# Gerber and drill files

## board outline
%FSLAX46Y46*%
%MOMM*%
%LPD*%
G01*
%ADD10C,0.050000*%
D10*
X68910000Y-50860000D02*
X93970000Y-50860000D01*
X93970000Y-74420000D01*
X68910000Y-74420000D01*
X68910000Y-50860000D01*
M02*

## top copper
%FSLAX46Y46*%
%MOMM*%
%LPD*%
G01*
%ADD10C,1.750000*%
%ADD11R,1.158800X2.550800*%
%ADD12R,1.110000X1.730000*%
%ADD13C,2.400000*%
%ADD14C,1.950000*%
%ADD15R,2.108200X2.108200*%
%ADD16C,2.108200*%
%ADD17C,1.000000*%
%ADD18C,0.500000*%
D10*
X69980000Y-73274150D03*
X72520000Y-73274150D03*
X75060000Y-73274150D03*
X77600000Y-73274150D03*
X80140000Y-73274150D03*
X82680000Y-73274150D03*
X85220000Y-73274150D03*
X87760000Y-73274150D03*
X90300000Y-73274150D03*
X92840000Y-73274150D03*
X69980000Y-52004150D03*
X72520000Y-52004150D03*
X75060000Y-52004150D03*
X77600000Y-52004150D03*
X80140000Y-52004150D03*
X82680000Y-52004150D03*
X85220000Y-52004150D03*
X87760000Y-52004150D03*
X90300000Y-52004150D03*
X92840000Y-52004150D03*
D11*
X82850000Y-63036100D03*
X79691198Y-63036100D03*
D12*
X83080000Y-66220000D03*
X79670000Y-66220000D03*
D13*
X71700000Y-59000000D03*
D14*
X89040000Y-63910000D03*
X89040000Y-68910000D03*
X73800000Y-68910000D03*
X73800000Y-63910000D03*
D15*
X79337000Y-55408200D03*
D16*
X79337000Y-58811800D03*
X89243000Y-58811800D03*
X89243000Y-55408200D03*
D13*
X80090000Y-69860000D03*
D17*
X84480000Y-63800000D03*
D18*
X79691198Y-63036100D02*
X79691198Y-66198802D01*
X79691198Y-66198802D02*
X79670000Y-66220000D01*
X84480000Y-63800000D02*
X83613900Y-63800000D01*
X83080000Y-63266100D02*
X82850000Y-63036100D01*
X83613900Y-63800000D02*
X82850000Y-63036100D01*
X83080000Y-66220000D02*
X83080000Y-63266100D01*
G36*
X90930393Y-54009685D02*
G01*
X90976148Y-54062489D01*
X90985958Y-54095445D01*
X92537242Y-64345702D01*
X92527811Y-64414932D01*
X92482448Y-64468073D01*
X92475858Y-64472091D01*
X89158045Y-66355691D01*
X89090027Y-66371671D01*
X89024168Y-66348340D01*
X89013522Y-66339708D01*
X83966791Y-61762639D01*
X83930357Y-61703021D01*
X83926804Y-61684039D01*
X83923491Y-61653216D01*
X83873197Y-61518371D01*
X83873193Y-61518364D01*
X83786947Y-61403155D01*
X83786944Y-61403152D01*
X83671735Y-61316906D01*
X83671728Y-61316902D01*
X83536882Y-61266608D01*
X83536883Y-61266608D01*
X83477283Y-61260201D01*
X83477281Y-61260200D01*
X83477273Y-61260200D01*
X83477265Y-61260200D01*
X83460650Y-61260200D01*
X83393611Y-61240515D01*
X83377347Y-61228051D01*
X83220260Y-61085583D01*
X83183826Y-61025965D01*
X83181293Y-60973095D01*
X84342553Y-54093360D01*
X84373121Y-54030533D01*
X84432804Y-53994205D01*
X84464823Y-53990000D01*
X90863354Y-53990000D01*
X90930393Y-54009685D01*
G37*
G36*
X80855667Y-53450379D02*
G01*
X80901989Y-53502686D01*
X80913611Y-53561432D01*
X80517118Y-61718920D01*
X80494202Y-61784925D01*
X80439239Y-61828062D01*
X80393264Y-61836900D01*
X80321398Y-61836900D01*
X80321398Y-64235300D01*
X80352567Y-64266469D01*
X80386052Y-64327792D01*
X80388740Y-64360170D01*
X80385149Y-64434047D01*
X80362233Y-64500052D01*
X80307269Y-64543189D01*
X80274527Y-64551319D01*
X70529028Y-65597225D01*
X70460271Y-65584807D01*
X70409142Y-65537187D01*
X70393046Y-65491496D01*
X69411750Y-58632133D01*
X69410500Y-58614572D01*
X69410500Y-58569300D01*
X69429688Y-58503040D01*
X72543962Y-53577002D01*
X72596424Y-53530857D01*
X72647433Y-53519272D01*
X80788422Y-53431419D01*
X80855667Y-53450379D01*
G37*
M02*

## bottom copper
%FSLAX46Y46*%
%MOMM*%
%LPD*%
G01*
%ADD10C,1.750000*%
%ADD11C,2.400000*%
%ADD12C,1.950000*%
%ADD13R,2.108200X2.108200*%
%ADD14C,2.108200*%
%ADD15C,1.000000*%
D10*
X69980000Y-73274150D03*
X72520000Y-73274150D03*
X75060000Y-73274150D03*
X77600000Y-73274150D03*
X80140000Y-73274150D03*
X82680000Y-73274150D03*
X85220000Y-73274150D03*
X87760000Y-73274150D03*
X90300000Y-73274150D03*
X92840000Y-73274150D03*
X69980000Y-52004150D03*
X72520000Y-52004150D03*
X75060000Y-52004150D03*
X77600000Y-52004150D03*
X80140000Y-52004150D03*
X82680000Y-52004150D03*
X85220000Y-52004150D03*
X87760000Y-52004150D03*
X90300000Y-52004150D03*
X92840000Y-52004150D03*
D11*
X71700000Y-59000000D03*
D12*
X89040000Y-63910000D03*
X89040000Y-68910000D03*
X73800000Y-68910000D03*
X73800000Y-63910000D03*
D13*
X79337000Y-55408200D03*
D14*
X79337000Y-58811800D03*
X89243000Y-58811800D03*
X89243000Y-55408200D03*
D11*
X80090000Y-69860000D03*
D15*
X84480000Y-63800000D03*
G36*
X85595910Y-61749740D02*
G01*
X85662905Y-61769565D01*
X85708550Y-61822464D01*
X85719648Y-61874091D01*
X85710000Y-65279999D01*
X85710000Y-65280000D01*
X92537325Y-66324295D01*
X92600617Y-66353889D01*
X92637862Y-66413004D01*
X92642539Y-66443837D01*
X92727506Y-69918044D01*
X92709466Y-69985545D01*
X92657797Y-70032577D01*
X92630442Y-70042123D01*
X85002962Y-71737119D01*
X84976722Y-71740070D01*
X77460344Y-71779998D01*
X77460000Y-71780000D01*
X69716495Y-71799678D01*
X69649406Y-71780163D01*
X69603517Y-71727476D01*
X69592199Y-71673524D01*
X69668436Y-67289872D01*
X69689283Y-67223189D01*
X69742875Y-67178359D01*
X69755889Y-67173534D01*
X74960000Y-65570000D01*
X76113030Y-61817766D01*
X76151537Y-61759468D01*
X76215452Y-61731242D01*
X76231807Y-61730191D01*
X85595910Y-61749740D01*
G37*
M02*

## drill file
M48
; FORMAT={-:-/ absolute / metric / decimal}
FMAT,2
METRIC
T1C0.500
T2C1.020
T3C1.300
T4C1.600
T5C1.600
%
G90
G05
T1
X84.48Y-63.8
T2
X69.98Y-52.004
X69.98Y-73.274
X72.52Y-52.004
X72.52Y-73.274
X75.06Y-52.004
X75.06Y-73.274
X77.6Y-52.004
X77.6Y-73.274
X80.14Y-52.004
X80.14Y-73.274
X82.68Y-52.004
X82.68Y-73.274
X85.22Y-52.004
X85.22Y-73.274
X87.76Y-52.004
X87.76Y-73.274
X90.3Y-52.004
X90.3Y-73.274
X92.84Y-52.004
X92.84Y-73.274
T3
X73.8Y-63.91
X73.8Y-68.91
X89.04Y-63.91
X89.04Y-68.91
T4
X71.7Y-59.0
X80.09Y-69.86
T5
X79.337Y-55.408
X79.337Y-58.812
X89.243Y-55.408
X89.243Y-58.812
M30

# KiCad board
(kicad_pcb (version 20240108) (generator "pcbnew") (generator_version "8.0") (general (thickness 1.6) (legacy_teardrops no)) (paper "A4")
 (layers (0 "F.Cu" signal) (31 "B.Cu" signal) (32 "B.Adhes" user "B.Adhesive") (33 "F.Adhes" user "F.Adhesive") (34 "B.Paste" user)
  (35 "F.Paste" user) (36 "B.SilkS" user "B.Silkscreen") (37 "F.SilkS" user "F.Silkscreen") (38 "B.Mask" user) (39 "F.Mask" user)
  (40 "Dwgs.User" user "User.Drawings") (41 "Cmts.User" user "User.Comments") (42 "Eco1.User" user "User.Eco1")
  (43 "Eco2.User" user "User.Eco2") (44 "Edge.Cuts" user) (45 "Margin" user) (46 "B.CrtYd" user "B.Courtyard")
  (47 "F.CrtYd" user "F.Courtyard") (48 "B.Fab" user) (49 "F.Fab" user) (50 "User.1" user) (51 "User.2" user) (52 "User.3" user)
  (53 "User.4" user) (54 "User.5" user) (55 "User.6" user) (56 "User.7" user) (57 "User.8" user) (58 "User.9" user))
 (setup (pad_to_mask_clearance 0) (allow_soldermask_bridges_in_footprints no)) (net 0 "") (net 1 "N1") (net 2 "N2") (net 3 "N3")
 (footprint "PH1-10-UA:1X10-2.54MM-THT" (layer "F.Cu") (at 69.98 73.27415)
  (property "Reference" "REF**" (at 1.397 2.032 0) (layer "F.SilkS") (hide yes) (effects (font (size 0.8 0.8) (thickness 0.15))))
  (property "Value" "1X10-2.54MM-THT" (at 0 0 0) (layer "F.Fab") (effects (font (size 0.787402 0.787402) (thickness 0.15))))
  (pad "1" thru_hole circle (at 0 0) (size 1.75 1.75) (drill 1.02) (layers "*.Cu" "*.Mask") (remove_unused_layers no)
   (solder_mask_margin 0.102))
  (pad "2" thru_hole circle (at 2.54 0) (size 1.75 1.75) (drill 1.02) (layers "*.Cu" "*.Mask") (remove_unused_layers no)
   (solder_mask_margin 0.102))
  (pad "3" thru_hole circle (at 5.08 0) (size 1.75 1.75) (drill 1.02) (layers "*.Cu" "*.Mask") (remove_unused_layers no)
   (solder_mask_margin 0.102))
  (pad "4" thru_hole circle (at 7.62 0) (size 1.75 1.75) (drill 1.02) (layers "*.Cu" "*.Mask") (remove_unused_layers no)
   (solder_mask_margin 0.102))
  (pad "5" thru_hole circle (at 10.16 0) (size 1.75 1.75) (drill 1.02) (layers "*.Cu" "*.Mask") (remove_unused_layers no)
   (solder_mask_margin 0.102))
  (pad "6" thru_hole circle (at 12.7 0) (size 1.75 1.75) (drill 1.02) (layers "*.Cu" "*.Mask") (remove_unused_layers no)
   (solder_mask_margin 0.102))
  (pad "7" thru_hole circle (at 15.24 0) (size 1.75 1.75) (drill 1.02) (layers "*.Cu" "*.Mask") (remove_unused_layers no)
   (solder_mask_margin 0.102))
  (pad "8" thru_hole circle (at 17.78 0) (size 1.75 1.75) (drill 1.02) (layers "*.Cu" "*.Mask") (remove_unused_layers no)
   (solder_mask_margin 0.102))
  (pad "9" thru_hole circle (at 20.32 0) (size 1.75 1.75) (drill 1.02) (layers "*.Cu" "*.Mask") (remove_unused_layers no)
   (solder_mask_margin 0.102))
  (pad "10" thru_hole circle (at 22.86 0) (size 1.75 1.75) (drill 1.02) (layers "*.Cu" "*.Mask") (remove_unused_layers no)
   (solder_mask_margin 0.102)))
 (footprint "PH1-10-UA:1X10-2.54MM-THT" (layer "F.Cu") (at 69.98 52.00415)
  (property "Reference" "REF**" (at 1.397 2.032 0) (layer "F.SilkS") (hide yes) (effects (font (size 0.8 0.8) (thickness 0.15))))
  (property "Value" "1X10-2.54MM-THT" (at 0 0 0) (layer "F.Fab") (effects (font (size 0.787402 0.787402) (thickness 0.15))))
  (pad "1" thru_hole circle (at 0 0) (size 1.75 1.75) (drill 1.02) (layers "*.Cu" "*.Mask") (remove_unused_layers no)
   (solder_mask_margin 0.102))
  (pad "2" thru_hole circle (at 2.54 0) (size 1.75 1.75) (drill 1.02) (layers "*.Cu" "*.Mask") (remove_unused_layers no)
   (solder_mask_margin 0.102))
  (pad "3" thru_hole circle (at 5.08 0) (size 1.75 1.75) (drill 1.02) (layers "*.Cu" "*.Mask") (remove_unused_layers no)
   (solder_mask_margin 0.102))
  (pad "4" thru_hole circle (at 7.62 0) (size 1.75 1.75) (drill 1.02) (layers "*.Cu" "*.Mask") (remove_unused_layers no)
   (solder_mask_margin 0.102))
  (pad "5" thru_hole circle (at 10.16 0) (size 1.75 1.75) (drill 1.02) (layers "*.Cu" "*.Mask") (remove_unused_layers no)
   (solder_mask_margin 0.102))
  (pad "6" thru_hole circle (at 12.7 0) (size 1.75 1.75) (drill 1.02) (layers "*.Cu" "*.Mask") (remove_unused_layers no)
   (solder_mask_margin 0.102))
  (pad "7" thru_hole circle (at 15.24 0) (size 1.75 1.75) (drill 1.02) (layers "*.Cu" "*.Mask") (remove_unused_layers no)
   (solder_mask_margin 0.102))
  (pad "8" thru_hole circle (at 17.78 0) (size 1.75 1.75) (drill 1.02) (layers "*.Cu" "*.Mask") (remove_unused_layers no)
   (solder_mask_margin 0.102))
  (pad "9" thru_hole circle (at 20.32 0) (size 1.75 1.75) (drill 1.02) (layers "*.Cu" "*.Mask") (remove_unused_layers no)
   (solder_mask_margin 0.102))
  (pad "10" thru_hole circle (at 22.86 0) (size 1.75 1.75) (drill 1.02) (layers "*.Cu" "*.Mask") (remove_unused_layers no)
   (solder_mask_margin 0.102)))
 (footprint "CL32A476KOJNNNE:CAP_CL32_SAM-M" (layer "F.Cu") (at 81.270599 63.0361 180)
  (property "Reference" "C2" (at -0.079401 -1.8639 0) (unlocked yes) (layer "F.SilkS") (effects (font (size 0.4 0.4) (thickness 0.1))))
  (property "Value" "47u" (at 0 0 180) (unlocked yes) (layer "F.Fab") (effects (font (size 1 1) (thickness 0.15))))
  (pad "1" smd rect (at -1.579401 0 180) (size 1.1588 2.5508) (layers "F.Cu" "F.Paste" "F.Mask") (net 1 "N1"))
  (pad "2" smd rect (at 1.579401 0 180) (size 1.1588 2.5508) (layers "F.Cu" "F.Paste" "F.Mask") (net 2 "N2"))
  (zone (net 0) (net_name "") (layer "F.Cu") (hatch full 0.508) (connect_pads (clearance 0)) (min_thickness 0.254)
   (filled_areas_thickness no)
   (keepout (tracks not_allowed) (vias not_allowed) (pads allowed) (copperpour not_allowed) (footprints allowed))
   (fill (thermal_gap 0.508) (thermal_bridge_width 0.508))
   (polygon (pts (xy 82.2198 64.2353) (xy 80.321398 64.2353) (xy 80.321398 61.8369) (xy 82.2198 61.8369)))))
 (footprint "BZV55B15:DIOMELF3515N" (layer "F.Cu") (at 81.375 66.22)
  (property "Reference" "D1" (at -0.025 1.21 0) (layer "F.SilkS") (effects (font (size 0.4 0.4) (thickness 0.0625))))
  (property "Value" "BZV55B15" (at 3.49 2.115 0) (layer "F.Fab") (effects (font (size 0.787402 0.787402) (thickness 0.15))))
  (pad "A" smd rect (at 1.705 0) (size 1.11 1.73) (layers "F.Cu" "F.Paste" "F.Mask") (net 1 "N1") (solder_mask_margin 0.102))
  (pad "C" smd rect (at -1.705 0) (size 1.11 1.73) (layers "F.Cu" "F.Paste" "F.Mask") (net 2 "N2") (solder_mask_margin 0.102)))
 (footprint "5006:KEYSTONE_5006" (layer "F.Cu") (at 71.7 59)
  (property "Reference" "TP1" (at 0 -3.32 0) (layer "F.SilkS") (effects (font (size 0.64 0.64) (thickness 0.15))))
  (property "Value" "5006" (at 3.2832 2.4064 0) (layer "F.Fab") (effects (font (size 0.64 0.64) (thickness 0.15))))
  (pad "TP" thru_hole circle (at 0 0) (size 2.4 2.4) (drill 1.6) (layers "*.Cu" "*.Mask") (remove_unused_layers no) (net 2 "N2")
   (solder_mask_margin 0.102)))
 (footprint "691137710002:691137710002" (layer "F.Cu") (at 89.04 66.41 -90)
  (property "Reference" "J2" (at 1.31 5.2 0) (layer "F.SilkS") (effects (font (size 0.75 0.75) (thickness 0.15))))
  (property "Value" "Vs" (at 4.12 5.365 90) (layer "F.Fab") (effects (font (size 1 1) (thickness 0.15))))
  (pad "1" thru_hole circle (at -2.5 0 270) (size 1.95 1.95) (drill 1.3) (layers "*.Cu" "*.Mask") (remove_unused_layers no) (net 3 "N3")
   (solder_mask_margin 0.102))
  (pad "2" thru_hole circle (at 2.5 0 270) (size 1.95 1.95) (drill 1.3) (layers "*.Cu" "*.Mask") (remove_unused_layers no) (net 1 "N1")
   (solder_mask_margin 0.102)))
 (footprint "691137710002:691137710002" (layer "F.Cu") (at 73.8 66.41 90)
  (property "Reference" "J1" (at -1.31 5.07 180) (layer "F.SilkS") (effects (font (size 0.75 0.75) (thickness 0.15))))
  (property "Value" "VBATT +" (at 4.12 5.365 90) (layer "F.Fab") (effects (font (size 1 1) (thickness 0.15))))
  (pad "1" thru_hole circle (at -2.5 0 90) (size 1.95 1.95) (drill 1.3) (layers "*.Cu" "*.Mask") (remove_unused_layers no) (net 1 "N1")
   (solder_mask_margin 0.102))
  (pad "2" thru_hole circle (at 2.5 0 90) (size 1.95 1.95) (drill 1.3) (layers "*.Cu" "*.Mask") (remove_unused_layers no) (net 2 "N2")
   (solder_mask_margin 0.102)))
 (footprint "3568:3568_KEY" (layer "F.Cu") (at 79.337 55.4082)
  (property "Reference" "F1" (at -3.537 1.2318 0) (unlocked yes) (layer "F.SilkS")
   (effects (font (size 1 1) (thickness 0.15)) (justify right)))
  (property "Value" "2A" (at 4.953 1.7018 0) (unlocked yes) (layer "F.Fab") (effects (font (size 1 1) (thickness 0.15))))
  (pad "1" thru_hole rect (at 0 0) (size 2.1082 2.1082) (drill 1.6002) (layers "*.Cu" "*.Mask") (remove_unused_layers no) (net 2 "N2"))
  (pad "2" thru_hole circle (at 0 3.4036) (size 2.1082 2.1082) (drill 1.6002) (layers "*.Cu" "*.Mask") (remove_unused_layers no)
   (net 2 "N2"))
  (pad "3" thru_hole circle (at 9.906 3.4036) (size 2.1082 2.1082) (drill 1.6002) (layers "*.Cu" "*.Mask") (remove_unused_layers no)
   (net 3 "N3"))
  (pad "4" thru_hole circle (at 9.906 0) (size 2.1082 2.1082) (drill 1.6002) (layers "*.Cu" "*.Mask") (remove_unused_layers no) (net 3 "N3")))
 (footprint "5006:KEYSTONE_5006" (layer "F.Cu") (at 80.09 69.86)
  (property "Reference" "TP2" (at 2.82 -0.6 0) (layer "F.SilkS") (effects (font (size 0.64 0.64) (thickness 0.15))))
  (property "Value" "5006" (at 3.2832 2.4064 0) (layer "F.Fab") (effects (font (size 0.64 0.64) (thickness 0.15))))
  (pad "TP" thru_hole circle (at 0 0) (size 2.4 2.4) (drill 1.6) (layers "*.Cu" "*.Mask") (remove_unused_layers no) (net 1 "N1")
   (solder_mask_margin 0.102)))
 (gr_rect (start 68.91 50.86) (end 93.97 74.42) (stroke (width 0.05) (type default)) (fill none) (layer "Edge.Cuts"))
 (segment (start 79.691198 63.0361) (end 79.691198 66.198802) (width 0.5) (layer "F.Cu") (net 2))
 (segment (start 79.691198 66.198802) (end 79.67 66.22) (width 0.5) (layer "F.Cu") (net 2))
 (segment (start 84.48 63.8) (end 83.6139 63.8) (width 0.5) (layer "F.Cu") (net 1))
 (segment (start 83.08 63.2661) (end 82.85 63.0361) (width 0.5) (layer "F.Cu") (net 1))
 (segment (start 83.6139 63.8) (end 82.85 63.0361) (width 0.5) (layer "F.Cu") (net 1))
 (segment (start 83.08 66.22) (end 83.08 63.2661) (width 0.5) (layer "F.Cu") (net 1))
 (via (at 84.48 63.8) (size 1) (drill 0.5) (layers "F.Cu" "B.Cu") (free yes) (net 1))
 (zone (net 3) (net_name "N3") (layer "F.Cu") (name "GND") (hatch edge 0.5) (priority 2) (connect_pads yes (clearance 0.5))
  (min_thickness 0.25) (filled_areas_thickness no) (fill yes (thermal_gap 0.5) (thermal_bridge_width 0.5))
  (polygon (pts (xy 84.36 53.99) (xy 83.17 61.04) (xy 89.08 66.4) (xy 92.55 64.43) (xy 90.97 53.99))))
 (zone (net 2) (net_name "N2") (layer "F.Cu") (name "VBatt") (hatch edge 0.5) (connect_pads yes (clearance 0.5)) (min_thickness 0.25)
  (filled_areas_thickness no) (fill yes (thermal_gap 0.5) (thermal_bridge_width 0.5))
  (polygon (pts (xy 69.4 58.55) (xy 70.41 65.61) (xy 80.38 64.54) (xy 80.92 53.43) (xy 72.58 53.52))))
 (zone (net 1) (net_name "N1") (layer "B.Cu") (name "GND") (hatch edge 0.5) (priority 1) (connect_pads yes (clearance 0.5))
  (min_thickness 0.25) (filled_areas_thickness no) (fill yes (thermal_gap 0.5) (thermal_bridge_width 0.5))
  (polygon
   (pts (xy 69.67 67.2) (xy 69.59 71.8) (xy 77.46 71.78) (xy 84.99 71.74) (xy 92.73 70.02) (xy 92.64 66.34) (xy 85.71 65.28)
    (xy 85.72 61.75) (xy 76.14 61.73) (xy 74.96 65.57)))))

